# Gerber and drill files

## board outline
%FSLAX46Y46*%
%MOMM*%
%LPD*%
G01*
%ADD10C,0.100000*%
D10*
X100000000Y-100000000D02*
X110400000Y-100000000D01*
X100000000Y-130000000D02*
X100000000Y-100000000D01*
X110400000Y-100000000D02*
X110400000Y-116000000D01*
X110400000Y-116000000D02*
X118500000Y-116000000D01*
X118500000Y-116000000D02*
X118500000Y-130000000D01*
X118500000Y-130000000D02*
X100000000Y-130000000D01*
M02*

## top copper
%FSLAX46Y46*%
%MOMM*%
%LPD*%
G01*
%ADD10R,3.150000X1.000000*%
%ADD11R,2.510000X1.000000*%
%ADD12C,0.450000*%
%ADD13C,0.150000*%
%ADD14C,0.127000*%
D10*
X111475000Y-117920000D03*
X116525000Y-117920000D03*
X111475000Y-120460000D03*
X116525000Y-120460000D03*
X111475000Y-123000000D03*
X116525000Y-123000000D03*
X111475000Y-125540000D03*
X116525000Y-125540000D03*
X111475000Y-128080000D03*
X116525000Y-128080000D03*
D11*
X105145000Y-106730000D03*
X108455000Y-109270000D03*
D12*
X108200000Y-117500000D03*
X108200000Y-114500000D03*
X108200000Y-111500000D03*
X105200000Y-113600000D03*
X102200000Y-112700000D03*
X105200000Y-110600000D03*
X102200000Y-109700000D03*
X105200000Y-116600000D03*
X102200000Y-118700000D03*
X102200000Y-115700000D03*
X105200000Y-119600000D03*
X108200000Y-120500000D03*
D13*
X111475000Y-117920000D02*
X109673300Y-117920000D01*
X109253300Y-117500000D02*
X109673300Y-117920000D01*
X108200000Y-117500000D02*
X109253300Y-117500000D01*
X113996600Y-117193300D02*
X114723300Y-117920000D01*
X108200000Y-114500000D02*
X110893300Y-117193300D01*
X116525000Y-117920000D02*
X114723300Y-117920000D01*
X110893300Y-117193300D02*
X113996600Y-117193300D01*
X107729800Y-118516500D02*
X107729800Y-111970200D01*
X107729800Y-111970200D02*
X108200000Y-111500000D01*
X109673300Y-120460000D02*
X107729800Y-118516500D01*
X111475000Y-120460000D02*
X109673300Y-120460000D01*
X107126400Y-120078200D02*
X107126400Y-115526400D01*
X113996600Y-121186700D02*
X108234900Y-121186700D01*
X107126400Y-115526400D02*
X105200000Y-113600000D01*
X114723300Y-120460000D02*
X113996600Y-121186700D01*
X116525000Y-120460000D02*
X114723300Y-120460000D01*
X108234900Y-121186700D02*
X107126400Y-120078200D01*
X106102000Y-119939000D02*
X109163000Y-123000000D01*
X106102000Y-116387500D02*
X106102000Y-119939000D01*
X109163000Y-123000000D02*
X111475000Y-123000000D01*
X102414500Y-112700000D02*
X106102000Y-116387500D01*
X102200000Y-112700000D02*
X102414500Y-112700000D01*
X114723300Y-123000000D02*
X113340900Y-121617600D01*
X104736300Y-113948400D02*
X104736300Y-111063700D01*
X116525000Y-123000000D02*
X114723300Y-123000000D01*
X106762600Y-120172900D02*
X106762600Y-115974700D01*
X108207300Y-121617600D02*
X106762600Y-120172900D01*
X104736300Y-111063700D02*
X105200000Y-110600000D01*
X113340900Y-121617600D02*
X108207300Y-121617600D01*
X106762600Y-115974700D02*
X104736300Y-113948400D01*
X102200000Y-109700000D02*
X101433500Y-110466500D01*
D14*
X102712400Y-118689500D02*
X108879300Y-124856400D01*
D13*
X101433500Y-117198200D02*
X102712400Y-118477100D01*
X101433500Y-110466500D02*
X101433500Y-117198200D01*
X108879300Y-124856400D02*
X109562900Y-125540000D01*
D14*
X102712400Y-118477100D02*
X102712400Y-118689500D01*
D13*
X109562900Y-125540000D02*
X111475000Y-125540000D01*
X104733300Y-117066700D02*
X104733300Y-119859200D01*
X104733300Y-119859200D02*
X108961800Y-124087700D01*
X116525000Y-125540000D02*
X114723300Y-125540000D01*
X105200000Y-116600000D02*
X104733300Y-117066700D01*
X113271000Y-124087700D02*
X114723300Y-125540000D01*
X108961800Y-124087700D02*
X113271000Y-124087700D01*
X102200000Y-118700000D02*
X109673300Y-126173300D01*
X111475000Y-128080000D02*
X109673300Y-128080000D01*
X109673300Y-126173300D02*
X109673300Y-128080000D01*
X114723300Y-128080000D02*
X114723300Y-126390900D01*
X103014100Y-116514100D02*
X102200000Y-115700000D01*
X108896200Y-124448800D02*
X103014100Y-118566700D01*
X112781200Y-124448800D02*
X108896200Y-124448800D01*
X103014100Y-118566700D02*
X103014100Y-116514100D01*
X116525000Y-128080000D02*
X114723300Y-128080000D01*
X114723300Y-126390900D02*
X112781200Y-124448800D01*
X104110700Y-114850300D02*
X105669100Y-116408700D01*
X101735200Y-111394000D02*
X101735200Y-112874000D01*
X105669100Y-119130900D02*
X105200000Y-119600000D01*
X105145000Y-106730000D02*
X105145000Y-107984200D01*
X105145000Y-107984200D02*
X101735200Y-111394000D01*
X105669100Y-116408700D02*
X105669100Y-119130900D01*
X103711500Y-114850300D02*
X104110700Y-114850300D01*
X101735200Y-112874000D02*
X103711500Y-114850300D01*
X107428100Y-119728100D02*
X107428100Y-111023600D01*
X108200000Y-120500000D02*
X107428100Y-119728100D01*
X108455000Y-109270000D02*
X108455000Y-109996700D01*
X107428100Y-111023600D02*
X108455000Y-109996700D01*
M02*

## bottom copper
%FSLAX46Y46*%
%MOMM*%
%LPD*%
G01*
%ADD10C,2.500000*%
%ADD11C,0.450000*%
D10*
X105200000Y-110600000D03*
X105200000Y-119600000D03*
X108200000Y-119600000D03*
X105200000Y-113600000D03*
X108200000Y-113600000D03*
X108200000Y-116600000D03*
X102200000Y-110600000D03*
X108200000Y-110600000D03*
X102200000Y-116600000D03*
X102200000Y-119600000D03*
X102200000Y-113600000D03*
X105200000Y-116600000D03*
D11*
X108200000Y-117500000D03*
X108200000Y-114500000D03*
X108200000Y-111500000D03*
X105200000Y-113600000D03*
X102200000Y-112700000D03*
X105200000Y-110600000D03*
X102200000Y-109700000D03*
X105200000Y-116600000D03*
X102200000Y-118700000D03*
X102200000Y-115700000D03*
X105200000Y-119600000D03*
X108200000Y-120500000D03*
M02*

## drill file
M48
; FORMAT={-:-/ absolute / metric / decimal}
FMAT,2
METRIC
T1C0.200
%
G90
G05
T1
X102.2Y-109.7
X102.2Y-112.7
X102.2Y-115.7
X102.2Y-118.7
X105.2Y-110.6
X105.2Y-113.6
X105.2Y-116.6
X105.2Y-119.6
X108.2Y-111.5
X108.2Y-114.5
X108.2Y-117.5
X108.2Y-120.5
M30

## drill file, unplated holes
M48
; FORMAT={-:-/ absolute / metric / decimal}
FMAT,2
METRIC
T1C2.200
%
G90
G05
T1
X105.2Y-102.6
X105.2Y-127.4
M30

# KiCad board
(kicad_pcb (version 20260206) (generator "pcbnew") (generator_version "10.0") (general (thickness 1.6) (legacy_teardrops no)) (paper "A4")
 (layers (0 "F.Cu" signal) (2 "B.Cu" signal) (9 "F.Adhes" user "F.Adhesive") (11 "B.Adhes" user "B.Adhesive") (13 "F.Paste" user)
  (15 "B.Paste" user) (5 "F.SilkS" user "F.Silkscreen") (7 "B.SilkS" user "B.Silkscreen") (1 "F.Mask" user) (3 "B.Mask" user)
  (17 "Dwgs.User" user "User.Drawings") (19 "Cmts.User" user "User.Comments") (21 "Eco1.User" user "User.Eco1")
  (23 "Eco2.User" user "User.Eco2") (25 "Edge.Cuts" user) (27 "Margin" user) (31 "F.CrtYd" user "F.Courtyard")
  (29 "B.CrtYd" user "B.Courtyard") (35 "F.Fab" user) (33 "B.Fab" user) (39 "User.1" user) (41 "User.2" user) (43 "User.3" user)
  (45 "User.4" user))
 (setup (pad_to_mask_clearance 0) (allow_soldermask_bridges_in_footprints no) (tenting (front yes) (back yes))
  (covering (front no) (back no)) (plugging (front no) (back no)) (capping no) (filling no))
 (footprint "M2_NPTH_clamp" (layer "F.Cu") (at 105.2 102.6)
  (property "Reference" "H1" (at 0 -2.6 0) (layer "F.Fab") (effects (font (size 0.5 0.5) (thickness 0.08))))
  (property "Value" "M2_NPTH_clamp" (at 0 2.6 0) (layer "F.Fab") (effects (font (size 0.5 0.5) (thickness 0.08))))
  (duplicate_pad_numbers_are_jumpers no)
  (pad "" np_thru_hole circle (at 0 0) (size 2.2 2.2) (drill 2.2) (layers "*.Cu" "*.Mask")))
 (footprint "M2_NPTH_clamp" (layer "F.Cu") (at 105.2 127.4)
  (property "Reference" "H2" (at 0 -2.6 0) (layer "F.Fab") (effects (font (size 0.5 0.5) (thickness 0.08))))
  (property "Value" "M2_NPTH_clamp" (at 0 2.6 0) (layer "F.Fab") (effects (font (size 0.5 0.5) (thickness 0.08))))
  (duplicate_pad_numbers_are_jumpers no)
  (pad "" np_thru_hole circle (at 0 0) (size 2.2 2.2) (drill 2.2) (layers "*.Cu" "*.Mask")))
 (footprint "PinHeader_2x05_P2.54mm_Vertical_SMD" (layer "F.Cu") (at 114 123)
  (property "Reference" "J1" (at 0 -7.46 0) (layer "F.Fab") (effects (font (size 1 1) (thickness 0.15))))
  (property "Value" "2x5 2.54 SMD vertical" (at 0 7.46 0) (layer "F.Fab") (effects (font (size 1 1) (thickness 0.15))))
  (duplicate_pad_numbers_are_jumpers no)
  (pad "1" smd rect (at -2.525 -5.08) (size 3.15 1) (layers "F.Cu" "F.Mask" "F.Paste") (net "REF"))
  (pad "2" smd rect (at 2.525 -5.08) (size 3.15 1) (layers "F.Cu" "F.Mask" "F.Paste") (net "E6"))
  (pad "3" smd rect (at -2.525 -2.54) (size 3.15 1) (layers "F.Cu" "F.Mask" "F.Paste") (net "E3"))
  (pad "4" smd rect (at 2.525 -2.54) (size 3.15 1) (layers "F.Cu" "F.Mask" "F.Paste") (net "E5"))
  (pad "5" smd rect (at -2.525 0) (size 3.15 1) (layers "F.Cu" "F.Mask" "F.Paste") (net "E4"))
  (pad "6" smd rect (at 2.525 0) (size 3.15 1) (layers "F.Cu" "F.Mask" "F.Paste") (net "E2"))
  (pad "7" smd rect (at -2.525 2.54) (size 3.15 1) (layers "F.Cu" "F.Mask" "F.Paste") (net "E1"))
  (pad "8" smd rect (at 2.525 2.54) (size 3.15 1) (layers "F.Cu" "F.Mask" "F.Paste") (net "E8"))
  (pad "9" smd rect (at -2.525 5.08) (size 3.15 1) (layers "F.Cu" "F.Mask" "F.Paste") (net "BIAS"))
  (pad "10" smd rect (at 2.525 5.08) (size 3.15 1) (layers "F.Cu" "F.Mask" "F.Paste") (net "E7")))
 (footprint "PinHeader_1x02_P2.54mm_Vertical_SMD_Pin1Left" (layer "F.Cu") (at 106.8 108)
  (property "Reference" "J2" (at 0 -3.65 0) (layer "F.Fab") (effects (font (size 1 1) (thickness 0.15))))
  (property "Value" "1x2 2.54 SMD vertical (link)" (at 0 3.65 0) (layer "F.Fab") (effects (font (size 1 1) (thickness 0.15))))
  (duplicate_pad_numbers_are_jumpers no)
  (pad "1" smd rect (at -1.655 -1.27) (size 2.51 1) (layers "F.Cu" "F.Mask" "F.Paste") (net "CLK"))
  (pad "2" smd rect (at 1.655 1.27) (size 2.51 1) (layers "F.Cu" "F.Mask" "F.Paste") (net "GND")))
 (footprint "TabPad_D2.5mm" (layer "B.Cu") (at 105.2 110.6 180)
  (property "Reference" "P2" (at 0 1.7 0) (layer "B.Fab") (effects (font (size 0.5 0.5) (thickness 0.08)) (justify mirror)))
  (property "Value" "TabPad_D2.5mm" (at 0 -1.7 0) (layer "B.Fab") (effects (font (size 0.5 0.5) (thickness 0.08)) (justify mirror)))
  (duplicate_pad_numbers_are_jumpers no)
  (pad "1" smd circle (at 0 0 180) (size 2.5 2.5) (layers "B.Cu" "B.Mask") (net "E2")))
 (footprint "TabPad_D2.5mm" (layer "B.Cu") (at 105.2 119.6 180)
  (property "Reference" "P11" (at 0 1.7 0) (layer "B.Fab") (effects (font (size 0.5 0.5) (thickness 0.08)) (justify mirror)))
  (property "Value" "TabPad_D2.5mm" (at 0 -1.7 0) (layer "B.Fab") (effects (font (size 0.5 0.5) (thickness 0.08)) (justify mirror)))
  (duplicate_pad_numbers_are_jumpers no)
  (pad "1" smd circle (at 0 0 180) (size 2.5 2.5) (layers "B.Cu" "B.Mask") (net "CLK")))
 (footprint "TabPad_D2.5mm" (layer "B.Cu") (at 108.2 119.6 180)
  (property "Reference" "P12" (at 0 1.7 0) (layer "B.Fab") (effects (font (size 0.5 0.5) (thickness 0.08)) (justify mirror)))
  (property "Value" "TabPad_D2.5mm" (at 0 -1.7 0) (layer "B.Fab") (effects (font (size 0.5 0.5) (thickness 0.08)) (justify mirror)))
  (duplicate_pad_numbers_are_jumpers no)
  (pad "1" smd circle (at 0 0 180) (size 2.5 2.5) (layers "B.Cu" "B.Mask") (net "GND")))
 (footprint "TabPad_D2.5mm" (layer "B.Cu") (at 105.2 113.6 180)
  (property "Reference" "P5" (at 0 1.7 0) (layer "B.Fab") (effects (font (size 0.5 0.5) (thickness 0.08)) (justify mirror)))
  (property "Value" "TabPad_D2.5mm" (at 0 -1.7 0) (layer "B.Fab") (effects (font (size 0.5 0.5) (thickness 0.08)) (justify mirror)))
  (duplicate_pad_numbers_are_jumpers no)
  (pad "1" smd circle (at 0 0 180) (size 2.5 2.5) (layers "B.Cu" "B.Mask") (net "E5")))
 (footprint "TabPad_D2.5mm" (layer "B.Cu") (at 108.2 113.6 180)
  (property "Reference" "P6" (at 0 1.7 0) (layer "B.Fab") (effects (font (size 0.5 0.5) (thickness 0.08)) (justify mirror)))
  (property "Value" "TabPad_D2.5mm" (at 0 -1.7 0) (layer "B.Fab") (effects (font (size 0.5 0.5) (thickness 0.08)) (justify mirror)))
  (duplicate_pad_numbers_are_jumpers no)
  (pad "1" smd circle (at 0 0 180) (size 2.5 2.5) (layers "B.Cu" "B.Mask") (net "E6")))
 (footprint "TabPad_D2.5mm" (layer "B.Cu") (at 108.2 116.6 180)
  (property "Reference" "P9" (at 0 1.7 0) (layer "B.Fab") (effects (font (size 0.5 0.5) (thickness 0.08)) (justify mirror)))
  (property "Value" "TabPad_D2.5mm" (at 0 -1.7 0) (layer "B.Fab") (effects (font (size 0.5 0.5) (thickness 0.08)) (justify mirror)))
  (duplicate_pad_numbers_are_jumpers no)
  (pad "1" smd circle (at 0 0 180) (size 2.5 2.5) (layers "B.Cu" "B.Mask") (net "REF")))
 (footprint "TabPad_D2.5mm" (layer "B.Cu") (at 102.2 110.6 180)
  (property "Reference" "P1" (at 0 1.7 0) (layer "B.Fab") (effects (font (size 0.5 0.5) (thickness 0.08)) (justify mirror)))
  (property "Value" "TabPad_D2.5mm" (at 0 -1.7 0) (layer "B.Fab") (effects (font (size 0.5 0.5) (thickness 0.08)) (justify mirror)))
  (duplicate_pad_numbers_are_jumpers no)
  (pad "1" smd circle (at 0 0 180) (size 2.5 2.5) (layers "B.Cu" "B.Mask") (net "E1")))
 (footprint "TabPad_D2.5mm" (layer "B.Cu") (at 108.2 110.6 180)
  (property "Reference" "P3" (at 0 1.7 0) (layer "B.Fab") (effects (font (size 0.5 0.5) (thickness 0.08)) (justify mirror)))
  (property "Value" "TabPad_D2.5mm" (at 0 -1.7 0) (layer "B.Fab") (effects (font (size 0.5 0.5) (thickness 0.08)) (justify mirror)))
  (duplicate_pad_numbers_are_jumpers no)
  (pad "1" smd circle (at 0 0 180) (size 2.5 2.5) (layers "B.Cu" "B.Mask") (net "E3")))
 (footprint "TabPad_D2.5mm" (layer "B.Cu") (at 102.2 116.6 180)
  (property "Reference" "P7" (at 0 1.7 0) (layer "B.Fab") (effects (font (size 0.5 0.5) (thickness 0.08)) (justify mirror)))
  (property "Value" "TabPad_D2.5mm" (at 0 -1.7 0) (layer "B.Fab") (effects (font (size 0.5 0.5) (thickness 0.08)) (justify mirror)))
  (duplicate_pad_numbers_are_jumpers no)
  (pad "1" smd circle (at 0 0 180) (size 2.5 2.5) (layers "B.Cu" "B.Mask") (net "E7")))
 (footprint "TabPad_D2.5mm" (layer "B.Cu") (at 102.2 119.6 180)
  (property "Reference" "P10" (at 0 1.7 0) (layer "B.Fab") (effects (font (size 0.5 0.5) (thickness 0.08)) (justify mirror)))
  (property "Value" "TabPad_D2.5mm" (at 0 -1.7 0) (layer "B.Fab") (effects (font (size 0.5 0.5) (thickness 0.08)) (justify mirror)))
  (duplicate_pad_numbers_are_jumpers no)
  (pad "1" smd circle (at 0 0 180) (size 2.5 2.5) (layers "B.Cu" "B.Mask") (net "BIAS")))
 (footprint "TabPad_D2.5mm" (layer "B.Cu") (at 102.2 113.6 180)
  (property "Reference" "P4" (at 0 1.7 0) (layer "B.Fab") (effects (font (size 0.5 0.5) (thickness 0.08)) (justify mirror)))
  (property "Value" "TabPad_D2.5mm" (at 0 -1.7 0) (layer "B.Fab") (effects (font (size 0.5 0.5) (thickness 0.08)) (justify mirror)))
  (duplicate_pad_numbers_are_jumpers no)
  (pad "1" smd circle (at 0 0 180) (size 2.5 2.5) (layers "B.Cu" "B.Mask") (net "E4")))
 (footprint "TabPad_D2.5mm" (layer "B.Cu") (at 105.2 116.6 180)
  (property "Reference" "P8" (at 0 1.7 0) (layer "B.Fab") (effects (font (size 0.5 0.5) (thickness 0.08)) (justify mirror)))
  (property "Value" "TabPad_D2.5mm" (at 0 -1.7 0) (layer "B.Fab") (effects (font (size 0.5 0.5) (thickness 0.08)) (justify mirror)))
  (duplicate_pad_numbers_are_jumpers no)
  (pad "1" smd circle (at 0 0 180) (size 2.5 2.5) (layers "B.Cu" "B.Mask") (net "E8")))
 (gr_line (start 100 100) (end 110.4 100) (stroke (width 0.1) (type default)) (layer "Edge.Cuts"))
 (gr_line (start 100 130) (end 100 100) (stroke (width 0.1) (type default)) (layer "Edge.Cuts"))
 (gr_line (start 110.4 100) (end 110.4 116) (stroke (width 0.1) (type default)) (layer "Edge.Cuts"))
 (gr_line (start 110.4 116) (end 118.5 116) (stroke (width 0.1) (type default)) (layer "Edge.Cuts"))
 (gr_line (start 118.5 116) (end 118.5 130) (stroke (width 0.1) (type default)) (layer "Edge.Cuts"))
 (gr_line (start 118.5 130) (end 100 130) (stroke (width 0.1) (type default)) (layer "Edge.Cuts"))
 (segment (start 111.475 117.92) (end 109.6733 117.92) (width 0.15) (layer "F.Cu") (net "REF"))
 (segment (start 109.2533 117.5) (end 109.6733 117.92) (width 0.15) (layer "F.Cu") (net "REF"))
 (segment (start 108.2 117.5) (end 109.2533 117.5) (width 0.15) (layer "F.Cu") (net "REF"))
 (via (at 108.2 117.5) (size 0.45) (drill 0.2) (layers "F.Cu" "B.Cu") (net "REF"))
 (segment (start 113.9966 117.1933) (end 114.7233 117.92) (width 0.15) (layer "F.Cu") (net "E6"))
 (segment (start 108.2 114.5) (end 110.8933 117.1933) (width 0.15) (layer "F.Cu") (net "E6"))
 (segment (start 116.525 117.92) (end 114.7233 117.92) (width 0.15) (layer "F.Cu") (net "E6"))
 (segment (start 110.8933 117.1933) (end 113.9966 117.1933) (width 0.15) (layer "F.Cu") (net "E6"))
 (via (at 108.2 114.5) (size 0.45) (drill 0.2) (layers "F.Cu" "B.Cu") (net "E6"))
 (segment (start 107.7298 118.5165) (end 107.7298 111.9702) (width 0.15) (layer "F.Cu") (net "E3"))
 (segment (start 107.7298 111.9702) (end 108.2 111.5) (width 0.15) (layer "F.Cu") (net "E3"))
 (segment (start 109.6733 120.46) (end 107.7298 118.5165) (width 0.15) (layer "F.Cu") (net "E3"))
 (segment (start 111.475 120.46) (end 109.6733 120.46) (width 0.15) (layer "F.Cu") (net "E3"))
 (via (at 108.2 111.5) (size 0.45) (drill 0.2) (layers "F.Cu" "B.Cu") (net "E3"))
 (segment (start 107.1264 120.0782) (end 107.1264 115.5264) (width 0.15) (layer "F.Cu") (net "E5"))
 (segment (start 113.9966 121.1867) (end 108.2349 121.1867) (width 0.15) (layer "F.Cu") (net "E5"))
 (segment (start 107.1264 115.5264) (end 105.2 113.6) (width 0.15) (layer "F.Cu") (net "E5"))
 (segment (start 114.7233 120.46) (end 113.9966 121.1867) (width 0.15) (layer "F.Cu") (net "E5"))
 (segment (start 116.525 120.46) (end 114.7233 120.46) (width 0.15) (layer "F.Cu") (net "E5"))
 (segment (start 108.2349 121.1867) (end 107.1264 120.0782) (width 0.15) (layer "F.Cu") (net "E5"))
 (via (at 105.2 113.6) (size 0.45) (drill 0.2) (layers "F.Cu" "B.Cu") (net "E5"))
 (segment (start 106.102 119.939) (end 109.163 123) (width 0.15) (layer "F.Cu") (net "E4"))
 (segment (start 106.102 116.3875) (end 106.102 119.939) (width 0.15) (layer "F.Cu") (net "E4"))
 (segment (start 109.163 123) (end 111.475 123) (width 0.15) (layer "F.Cu") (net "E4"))
 (segment (start 102.4145 112.7) (end 106.102 116.3875) (width 0.15) (layer "F.Cu") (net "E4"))
 (segment (start 102.2 112.7) (end 102.4145 112.7) (width 0.15) (layer "F.Cu") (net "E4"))
 (via (at 102.2 112.7) (size 0.45) (drill 0.2) (layers "F.Cu" "B.Cu") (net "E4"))
 (segment (start 114.7233 123) (end 113.3409 121.6176) (width 0.15) (layer "F.Cu") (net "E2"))
 (segment (start 104.7363 113.9484) (end 104.7363 111.0637) (width 0.15) (layer "F.Cu") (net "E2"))
 (segment (start 116.525 123) (end 114.7233 123) (width 0.15) (layer "F.Cu") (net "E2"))
 (segment (start 106.7626 120.1729) (end 106.7626 115.9747) (width 0.15) (layer "F.Cu") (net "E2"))
 (segment (start 108.2073 121.6176) (end 106.7626 120.1729) (width 0.15) (layer "F.Cu") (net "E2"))
 (segment (start 104.7363 111.0637) (end 105.2 110.6) (width 0.15) (layer "F.Cu") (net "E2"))
 (segment (start 113.3409 121.6176) (end 108.2073 121.6176) (width 0.15) (layer "F.Cu") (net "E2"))
 (segment (start 106.7626 115.9747) (end 104.7363 113.9484) (width 0.15) (layer "F.Cu") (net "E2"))
 (via (at 105.2 110.6) (size 0.45) (drill 0.2) (layers "F.Cu" "B.Cu") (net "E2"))
 (segment (start 102.2 109.7) (end 101.4335 110.4665) (width 0.15) (layer "F.Cu") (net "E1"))
 (segment (start 102.7124 118.6895) (end 108.8793 124.8564) (width 0.127) (layer "F.Cu") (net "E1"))
 (segment (start 101.4335 117.1982) (end 102.7124 118.4771) (width 0.15) (layer "F.Cu") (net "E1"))
 (segment (start 101.4335 110.4665) (end 101.4335 117.1982) (width 0.15) (layer "F.Cu") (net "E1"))
 (segment (start 108.8793 124.8564) (end 109.5629 125.54) (width 0.15) (layer "F.Cu") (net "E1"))
 (segment (start 102.7124 118.4771) (end 102.7124 118.6895) (width 0.127) (layer "F.Cu") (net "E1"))
 (segment (start 109.5629 125.54) (end 111.475 125.54) (width 0.15) (layer "F.Cu") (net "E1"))
 (via (at 102.2 109.7) (size 0.45) (drill 0.2) (layers "F.Cu" "B.Cu") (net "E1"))
 (segment (start 104.7333 117.0667) (end 104.7333 119.8592) (width 0.15) (layer "F.Cu") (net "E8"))
 (segment (start 104.7333 119.8592) (end 108.9618 124.0877) (width 0.15) (layer "F.Cu") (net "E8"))
 (segment (start 116.525 125.54) (end 114.7233 125.54) (width 0.15) (layer "F.Cu") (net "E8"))
 (segment (start 105.2 116.6) (end 104.7333 117.0667) (width 0.15) (layer "F.Cu") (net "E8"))
 (segment (start 113.271 124.0877) (end 114.7233 125.54) (width 0.15) (layer "F.Cu") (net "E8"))
 (segment (start 108.9618 124.0877) (end 113.271 124.0877) (width 0.15) (layer "F.Cu") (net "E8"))
 (via (at 105.2 116.6) (size 0.45) (drill 0.2) (layers "F.Cu" "B.Cu") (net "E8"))
 (segment (start 102.2 118.7) (end 109.6733 126.1733) (width 0.15) (layer "F.Cu") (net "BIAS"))
 (segment (start 111.475 128.08) (end 109.6733 128.08) (width 0.15) (layer "F.Cu") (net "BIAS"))
 (segment (start 109.6733 126.1733) (end 109.6733 128.08) (width 0.15) (layer "F.Cu") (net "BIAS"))
 (via (at 102.2 118.7) (size 0.45) (drill 0.2) (layers "F.Cu" "B.Cu") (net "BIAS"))
 (segment (start 114.7233 128.08) (end 114.7233 126.3909) (width 0.15) (layer "F.Cu") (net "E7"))
 (segment (start 103.0141 116.5141) (end 102.2 115.7) (width 0.15) (layer "F.Cu") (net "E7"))
 (segment (start 108.8962 124.4488) (end 103.0141 118.5667) (width 0.15) (layer "F.Cu") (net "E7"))
 (segment (start 112.7812 124.4488) (end 108.8962 124.4488) (width 0.15) (layer "F.Cu") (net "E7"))
 (segment (start 103.0141 118.5667) (end 103.0141 116.5141) (width 0.15) (layer "F.Cu") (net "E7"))
 (segment (start 116.525 128.08) (end 114.7233 128.08) (width 0.15) (layer "F.Cu") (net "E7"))
 (segment (start 114.7233 126.3909) (end 112.7812 124.4488) (width 0.15) (layer "F.Cu") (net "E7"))
 (via (at 102.2 115.7) (size 0.45) (drill 0.2) (layers "F.Cu" "B.Cu") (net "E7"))
 (segment (start 104.1107 114.8503) (end 105.6691 116.4087) (width 0.15) (layer "F.Cu") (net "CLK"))
 (segment (start 101.7352 111.394) (end 101.7352 112.874) (width 0.15) (layer "F.Cu") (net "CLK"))
 (segment (start 105.6691 119.1309) (end 105.2 119.6) (width 0.15) (layer "F.Cu") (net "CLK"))
 (segment (start 105.145 106.73) (end 105.145 107.9842) (width 0.15) (layer "F.Cu") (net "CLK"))
 (segment (start 105.145 107.9842) (end 101.7352 111.394) (width 0.15) (layer "F.Cu") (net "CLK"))
 (segment (start 105.6691 116.4087) (end 105.6691 119.1309) (width 0.15) (layer "F.Cu") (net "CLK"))
 (segment (start 103.7115 114.8503) (end 104.1107 114.8503) (width 0.15) (layer "F.Cu") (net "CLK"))
 (segment (start 101.7352 112.874) (end 103.7115 114.8503) (width 0.15) (layer "F.Cu") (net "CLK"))
 (via (at 105.2 119.6) (size 0.45) (drill 0.2) (layers "F.Cu" "B.Cu") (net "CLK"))
 (segment (start 107.4281 119.7281) (end 107.4281 111.0236) (width 0.15) (layer "F.Cu") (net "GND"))
 (segment (start 108.2 120.5) (end 107.4281 119.7281) (width 0.15) (layer "F.Cu") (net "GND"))
 (segment (start 108.455 109.27) (end 108.455 109.9967) (width 0.15) (layer "F.Cu") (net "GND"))
 (segment (start 107.4281 111.0236) (end 108.455 109.9967) (width 0.15) (layer "F.Cu") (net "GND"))
 (via (at 108.2 120.5) (size 0.45) (drill 0.2) (layers "F.Cu" "B.Cu") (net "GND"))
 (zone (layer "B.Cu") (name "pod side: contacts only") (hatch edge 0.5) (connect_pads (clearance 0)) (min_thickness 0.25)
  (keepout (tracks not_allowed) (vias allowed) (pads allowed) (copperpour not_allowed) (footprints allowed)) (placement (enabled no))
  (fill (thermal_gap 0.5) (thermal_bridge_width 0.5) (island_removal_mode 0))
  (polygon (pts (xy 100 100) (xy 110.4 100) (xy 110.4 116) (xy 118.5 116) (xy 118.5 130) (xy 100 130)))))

